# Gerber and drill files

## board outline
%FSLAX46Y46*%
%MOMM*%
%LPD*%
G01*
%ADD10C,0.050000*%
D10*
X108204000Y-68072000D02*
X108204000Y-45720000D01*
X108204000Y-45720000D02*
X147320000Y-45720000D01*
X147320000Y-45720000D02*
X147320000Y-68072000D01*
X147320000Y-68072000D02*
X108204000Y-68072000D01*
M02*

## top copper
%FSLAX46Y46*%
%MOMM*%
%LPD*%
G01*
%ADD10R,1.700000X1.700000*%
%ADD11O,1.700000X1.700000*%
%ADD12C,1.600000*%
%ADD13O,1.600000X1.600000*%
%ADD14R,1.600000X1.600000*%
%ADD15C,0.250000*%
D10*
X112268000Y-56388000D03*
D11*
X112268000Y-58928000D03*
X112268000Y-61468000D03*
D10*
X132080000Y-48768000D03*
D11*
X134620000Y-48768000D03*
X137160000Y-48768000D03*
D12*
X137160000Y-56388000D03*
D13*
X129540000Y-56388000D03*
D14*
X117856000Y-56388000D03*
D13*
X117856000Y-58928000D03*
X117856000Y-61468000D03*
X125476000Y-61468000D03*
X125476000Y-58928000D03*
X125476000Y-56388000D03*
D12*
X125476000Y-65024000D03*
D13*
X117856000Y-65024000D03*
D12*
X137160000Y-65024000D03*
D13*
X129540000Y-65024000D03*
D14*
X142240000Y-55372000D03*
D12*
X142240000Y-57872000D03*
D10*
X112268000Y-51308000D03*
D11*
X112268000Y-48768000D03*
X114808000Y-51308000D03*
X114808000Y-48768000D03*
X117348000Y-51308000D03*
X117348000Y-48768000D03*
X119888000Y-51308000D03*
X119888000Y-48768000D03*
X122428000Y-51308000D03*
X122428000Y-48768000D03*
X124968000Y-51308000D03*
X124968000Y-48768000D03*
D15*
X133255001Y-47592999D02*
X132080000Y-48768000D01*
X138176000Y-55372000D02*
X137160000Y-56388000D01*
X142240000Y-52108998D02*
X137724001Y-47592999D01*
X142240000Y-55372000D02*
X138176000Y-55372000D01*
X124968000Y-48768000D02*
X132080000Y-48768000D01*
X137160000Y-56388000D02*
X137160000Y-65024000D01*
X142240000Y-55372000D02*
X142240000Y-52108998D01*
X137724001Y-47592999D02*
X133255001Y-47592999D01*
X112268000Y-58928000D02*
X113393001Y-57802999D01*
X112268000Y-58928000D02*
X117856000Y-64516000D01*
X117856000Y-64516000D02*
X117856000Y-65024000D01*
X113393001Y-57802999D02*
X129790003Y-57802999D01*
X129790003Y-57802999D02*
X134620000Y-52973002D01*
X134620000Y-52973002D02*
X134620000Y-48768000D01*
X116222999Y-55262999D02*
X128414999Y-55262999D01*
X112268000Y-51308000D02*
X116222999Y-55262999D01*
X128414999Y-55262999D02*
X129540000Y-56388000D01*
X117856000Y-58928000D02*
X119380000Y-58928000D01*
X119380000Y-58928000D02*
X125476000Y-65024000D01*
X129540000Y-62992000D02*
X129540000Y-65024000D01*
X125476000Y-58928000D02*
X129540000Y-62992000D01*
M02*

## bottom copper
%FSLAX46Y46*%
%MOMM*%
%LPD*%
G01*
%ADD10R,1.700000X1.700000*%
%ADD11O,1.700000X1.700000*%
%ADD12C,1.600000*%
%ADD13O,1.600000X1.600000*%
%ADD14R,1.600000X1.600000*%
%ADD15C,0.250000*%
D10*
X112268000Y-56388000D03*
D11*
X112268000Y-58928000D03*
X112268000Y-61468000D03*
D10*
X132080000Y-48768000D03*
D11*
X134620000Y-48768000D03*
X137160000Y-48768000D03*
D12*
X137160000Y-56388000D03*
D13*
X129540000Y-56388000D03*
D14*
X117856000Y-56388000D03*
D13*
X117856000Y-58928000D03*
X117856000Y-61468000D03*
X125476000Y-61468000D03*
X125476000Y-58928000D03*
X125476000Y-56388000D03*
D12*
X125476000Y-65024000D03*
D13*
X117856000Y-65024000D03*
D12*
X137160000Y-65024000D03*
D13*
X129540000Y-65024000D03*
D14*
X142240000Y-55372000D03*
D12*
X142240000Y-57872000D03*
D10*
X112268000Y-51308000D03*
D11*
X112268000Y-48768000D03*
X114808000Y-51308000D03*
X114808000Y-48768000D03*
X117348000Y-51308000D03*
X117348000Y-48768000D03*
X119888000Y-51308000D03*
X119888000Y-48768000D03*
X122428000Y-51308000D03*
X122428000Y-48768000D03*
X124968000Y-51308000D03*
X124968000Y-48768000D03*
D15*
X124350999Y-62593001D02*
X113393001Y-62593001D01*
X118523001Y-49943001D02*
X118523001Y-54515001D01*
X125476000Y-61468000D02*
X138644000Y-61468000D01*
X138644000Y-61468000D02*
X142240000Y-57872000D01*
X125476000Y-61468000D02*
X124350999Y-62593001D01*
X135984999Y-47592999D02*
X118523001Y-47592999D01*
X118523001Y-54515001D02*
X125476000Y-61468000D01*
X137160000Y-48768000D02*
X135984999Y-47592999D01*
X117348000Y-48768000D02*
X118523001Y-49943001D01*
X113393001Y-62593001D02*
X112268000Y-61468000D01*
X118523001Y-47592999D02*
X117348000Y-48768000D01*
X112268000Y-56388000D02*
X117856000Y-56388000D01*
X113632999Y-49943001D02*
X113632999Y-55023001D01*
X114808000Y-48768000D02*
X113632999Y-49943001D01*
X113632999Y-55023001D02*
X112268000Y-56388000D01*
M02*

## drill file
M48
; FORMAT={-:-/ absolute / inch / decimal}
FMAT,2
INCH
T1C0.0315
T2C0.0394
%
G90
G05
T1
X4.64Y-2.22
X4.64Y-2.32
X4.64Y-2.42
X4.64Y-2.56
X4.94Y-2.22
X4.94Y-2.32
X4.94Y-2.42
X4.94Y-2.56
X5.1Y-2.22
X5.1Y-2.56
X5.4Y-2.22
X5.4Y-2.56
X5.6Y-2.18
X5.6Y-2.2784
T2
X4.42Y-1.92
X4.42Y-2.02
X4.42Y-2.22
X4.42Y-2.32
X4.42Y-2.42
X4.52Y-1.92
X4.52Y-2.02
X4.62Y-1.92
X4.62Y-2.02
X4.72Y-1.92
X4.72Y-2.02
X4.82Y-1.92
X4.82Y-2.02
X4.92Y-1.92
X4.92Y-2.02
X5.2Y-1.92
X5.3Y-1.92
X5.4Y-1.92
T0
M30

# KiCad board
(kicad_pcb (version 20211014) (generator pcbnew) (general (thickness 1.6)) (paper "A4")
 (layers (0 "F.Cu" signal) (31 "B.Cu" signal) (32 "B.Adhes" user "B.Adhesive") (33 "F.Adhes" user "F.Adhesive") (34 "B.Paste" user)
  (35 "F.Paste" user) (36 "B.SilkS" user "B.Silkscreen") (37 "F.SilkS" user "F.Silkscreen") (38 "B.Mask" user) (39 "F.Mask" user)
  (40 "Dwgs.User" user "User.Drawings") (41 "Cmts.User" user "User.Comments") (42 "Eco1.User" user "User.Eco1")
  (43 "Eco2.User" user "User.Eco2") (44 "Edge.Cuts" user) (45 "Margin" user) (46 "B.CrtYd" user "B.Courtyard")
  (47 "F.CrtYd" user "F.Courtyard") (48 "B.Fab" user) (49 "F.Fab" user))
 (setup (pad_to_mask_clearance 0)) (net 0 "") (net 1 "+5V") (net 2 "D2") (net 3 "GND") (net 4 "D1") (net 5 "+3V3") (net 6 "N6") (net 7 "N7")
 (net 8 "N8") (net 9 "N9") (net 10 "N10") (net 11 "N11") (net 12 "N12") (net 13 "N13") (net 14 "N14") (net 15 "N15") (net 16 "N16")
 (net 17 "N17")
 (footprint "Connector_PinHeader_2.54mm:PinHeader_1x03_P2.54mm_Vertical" (layer "F.Cu") (at 112.268 56.388)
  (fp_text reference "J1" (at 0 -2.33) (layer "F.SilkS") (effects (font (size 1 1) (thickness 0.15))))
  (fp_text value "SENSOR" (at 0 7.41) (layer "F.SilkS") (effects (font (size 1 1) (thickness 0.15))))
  (pad "1" thru_hole rect locked (at 0 0) (size 1.7 1.7) (drill 1) (layers *.Cu *.Mask) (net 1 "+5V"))
  (pad "2" thru_hole oval locked (at 0 2.54) (size 1.7 1.7) (drill 1) (layers *.Cu *.Mask) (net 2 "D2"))
  (pad "3" thru_hole oval locked (at 0 5.08) (size 1.7 1.7) (drill 1) (layers *.Cu *.Mask) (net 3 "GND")))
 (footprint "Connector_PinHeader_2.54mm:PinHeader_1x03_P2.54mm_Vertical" (layer "F.Cu") (at 132.08 48.768 90)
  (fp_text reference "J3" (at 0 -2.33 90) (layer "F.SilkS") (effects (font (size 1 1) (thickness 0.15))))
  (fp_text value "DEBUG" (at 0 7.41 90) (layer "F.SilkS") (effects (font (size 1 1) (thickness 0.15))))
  (pad "1" thru_hole rect locked (at 0 0 90) (size 1.7 1.7) (drill 1) (layers *.Cu *.Mask) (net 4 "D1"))
  (pad "2" thru_hole oval locked (at 0 2.54 90) (size 1.7 1.7) (drill 1) (layers *.Cu *.Mask) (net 2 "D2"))
  (pad "3" thru_hole oval locked (at 0 5.08 90) (size 1.7 1.7) (drill 1) (layers *.Cu *.Mask) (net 3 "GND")))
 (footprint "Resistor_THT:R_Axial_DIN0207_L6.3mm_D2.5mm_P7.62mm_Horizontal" (layer "F.Cu") (at 137.16 56.388 180)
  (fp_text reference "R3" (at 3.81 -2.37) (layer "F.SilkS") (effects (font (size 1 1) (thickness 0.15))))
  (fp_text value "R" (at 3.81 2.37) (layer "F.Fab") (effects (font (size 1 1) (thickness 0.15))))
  (pad "1" thru_hole circle locked (at 0 0 180) (size 1.6 1.6) (drill 0.8) (layers *.Cu *.Mask) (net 4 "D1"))
  (pad "2" thru_hole oval locked (at 7.62 0 180) (size 1.6 1.6) (drill 0.8) (layers *.Cu *.Mask) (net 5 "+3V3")))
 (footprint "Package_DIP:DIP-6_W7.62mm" (layer "F.Cu") (at 117.856 56.388)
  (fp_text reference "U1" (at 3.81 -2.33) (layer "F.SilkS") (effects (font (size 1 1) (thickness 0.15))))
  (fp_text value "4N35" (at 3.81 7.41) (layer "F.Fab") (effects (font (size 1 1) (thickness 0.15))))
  (pad "1" thru_hole rect locked (at 0 0) (size 1.6 1.6) (drill 0.8) (layers *.Cu *.Mask) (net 1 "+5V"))
  (pad "2" thru_hole oval locked (at 0 2.54) (size 1.6 1.6) (drill 0.8) (layers *.Cu *.Mask) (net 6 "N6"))
  (pad "3" thru_hole oval locked (at 0 5.08) (size 1.6 1.6) (drill 0.8) (layers *.Cu *.Mask) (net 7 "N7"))
  (pad "4" thru_hole oval locked (at 7.62 5.08) (size 1.6 1.6) (drill 0.8) (layers *.Cu *.Mask) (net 3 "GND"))
  (pad "5" thru_hole oval locked (at 7.62 2.54) (size 1.6 1.6) (drill 0.8) (layers *.Cu *.Mask) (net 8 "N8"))
  (pad "6" thru_hole oval locked (at 7.62 0) (size 1.6 1.6) (drill 0.8) (layers *.Cu *.Mask) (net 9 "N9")))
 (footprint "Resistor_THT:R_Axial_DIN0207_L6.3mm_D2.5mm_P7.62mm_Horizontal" (layer "F.Cu") (at 125.476 65.024 180)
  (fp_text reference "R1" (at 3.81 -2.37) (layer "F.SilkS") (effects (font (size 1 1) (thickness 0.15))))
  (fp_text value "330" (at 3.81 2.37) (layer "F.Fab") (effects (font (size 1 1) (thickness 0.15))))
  (pad "1" thru_hole circle locked (at 0 0 180) (size 1.6 1.6) (drill 0.8) (layers *.Cu *.Mask) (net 6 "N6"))
  (pad "2" thru_hole oval locked (at 7.62 0 180) (size 1.6 1.6) (drill 0.8) (layers *.Cu *.Mask) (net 2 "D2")))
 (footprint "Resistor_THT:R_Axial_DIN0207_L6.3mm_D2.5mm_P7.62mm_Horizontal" (layer "F.Cu") (at 137.16 65.024 180)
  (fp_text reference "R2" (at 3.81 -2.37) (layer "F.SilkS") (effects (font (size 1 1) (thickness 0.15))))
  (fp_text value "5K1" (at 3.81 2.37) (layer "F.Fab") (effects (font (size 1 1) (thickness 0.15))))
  (pad "1" thru_hole circle locked (at 0 0 180) (size 1.6 1.6) (drill 0.8) (layers *.Cu *.Mask) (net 4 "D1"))
  (pad "2" thru_hole oval locked (at 7.62 0 180) (size 1.6 1.6) (drill 0.8) (layers *.Cu *.Mask) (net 8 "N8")))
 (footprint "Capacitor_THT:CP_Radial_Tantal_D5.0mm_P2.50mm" (layer "F.Cu") (at 142.24 55.372 -90)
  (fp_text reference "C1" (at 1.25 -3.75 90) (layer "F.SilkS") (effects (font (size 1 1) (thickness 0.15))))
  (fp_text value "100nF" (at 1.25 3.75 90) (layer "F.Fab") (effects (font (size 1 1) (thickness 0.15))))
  (pad "1" thru_hole rect locked (at 0 0 270) (size 1.6 1.6) (drill 0.8) (layers *.Cu *.Mask) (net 4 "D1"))
  (pad "2" thru_hole circle locked (at 2.5 0 270) (size 1.6 1.6) (drill 0.8) (layers *.Cu *.Mask) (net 3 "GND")))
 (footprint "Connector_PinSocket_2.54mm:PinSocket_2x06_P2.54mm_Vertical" (layer "B.Cu") (at 112.268 51.308 -90)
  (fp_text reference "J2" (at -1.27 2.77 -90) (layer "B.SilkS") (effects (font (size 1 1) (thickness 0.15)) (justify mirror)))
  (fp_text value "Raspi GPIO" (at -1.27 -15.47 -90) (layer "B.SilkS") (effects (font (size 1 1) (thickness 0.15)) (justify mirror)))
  (pad "1" thru_hole rect locked (at 0 0 270) (size 1.7 1.7) (drill 1) (layers *.Cu *.Mask) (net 5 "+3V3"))
  (pad "2" thru_hole oval locked (at -2.54 0 270) (size 1.7 1.7) (drill 1) (layers *.Cu *.Mask) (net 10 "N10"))
  (pad "3" thru_hole oval locked (at 0 -2.54 270) (size 1.7 1.7) (drill 1) (layers *.Cu *.Mask) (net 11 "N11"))
  (pad "4" thru_hole oval locked (at -2.54 -2.54 270) (size 1.7 1.7) (drill 1) (layers *.Cu *.Mask) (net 1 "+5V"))
  (pad "5" thru_hole oval locked (at 0 -5.08 270) (size 1.7 1.7) (drill 1) (layers *.Cu *.Mask) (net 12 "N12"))
  (pad "6" thru_hole oval locked (at -2.54 -5.08 270) (size 1.7 1.7) (drill 1) (layers *.Cu *.Mask) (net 3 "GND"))
  (pad "7" thru_hole oval locked (at 0 -7.62 270) (size 1.7 1.7) (drill 1) (layers *.Cu *.Mask) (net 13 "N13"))
  (pad "8" thru_hole oval locked (at -2.54 -7.62 270) (size 1.7 1.7) (drill 1) (layers *.Cu *.Mask) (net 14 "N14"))
  (pad "9" thru_hole oval locked (at 0 -10.16 270) (size 1.7 1.7) (drill 1) (layers *.Cu *.Mask) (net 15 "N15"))
  (pad "10" thru_hole oval locked (at -2.54 -10.16 270) (size 1.7 1.7) (drill 1) (layers *.Cu *.Mask) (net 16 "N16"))
  (pad "11" thru_hole oval locked (at 0 -12.7 270) (size 1.7 1.7) (drill 1) (layers *.Cu *.Mask) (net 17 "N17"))
  (pad "12" thru_hole oval locked (at -2.54 -12.7 270) (size 1.7 1.7) (drill 1) (layers *.Cu *.Mask) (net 4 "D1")))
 (gr_line (start 108.204 68.072) (end 108.204 45.72) (layer "Edge.Cuts") (width 0.05))
 (gr_line (start 108.204 45.72) (end 147.32 45.72) (layer "Edge.Cuts") (width 0.05))
 (gr_line (start 147.32 45.72) (end 147.32 68.072) (layer "Edge.Cuts") (width 0.05))
 (gr_line (start 147.32 68.072) (end 108.204 68.072) (layer "Edge.Cuts") (width 0.05))
 (segment (start 124.350999 62.593001) (end 113.393001 62.593001) (width 0.25) (layer "B.Cu") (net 3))
 (segment (start 118.523001 49.943001) (end 118.523001 54.515001) (width 0.25) (layer "B.Cu") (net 3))
 (segment (start 125.476 61.468) (end 138.644 61.468) (width 0.25) (layer "B.Cu") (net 3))
 (segment (start 138.644 61.468) (end 142.24 57.872) (width 0.25) (layer "B.Cu") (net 3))
 (segment (start 125.476 61.468) (end 124.350999 62.593001) (width 0.25) (layer "B.Cu") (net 3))
 (segment (start 135.984999 47.592999) (end 118.523001 47.592999) (width 0.25) (layer "B.Cu") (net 3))
 (segment (start 118.523001 54.515001) (end 125.476 61.468) (width 0.25) (layer "B.Cu") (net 3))
 (segment (start 137.16 48.768) (end 135.984999 47.592999) (width 0.25) (layer "B.Cu") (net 3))
 (segment (start 117.348 48.768) (end 118.523001 49.943001) (width 0.25) (layer "B.Cu") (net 3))
 (segment (start 113.393001 62.593001) (end 112.268 61.468) (width 0.25) (layer "B.Cu") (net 3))
 (segment (start 118.523001 47.592999) (end 117.348 48.768) (width 0.25) (layer "B.Cu") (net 3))
 (segment (start 133.255001 47.592999) (end 132.08 48.768) (width 0.25) (layer "F.Cu") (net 4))
 (segment (start 138.176 55.372) (end 137.16 56.388) (width 0.25) (layer "F.Cu") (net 4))
 (segment (start 142.24 52.108998) (end 137.724001 47.592999) (width 0.25) (layer "F.Cu") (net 4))
 (segment (start 142.24 55.372) (end 138.176 55.372) (width 0.25) (layer "F.Cu") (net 4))
 (segment (start 124.968 48.768) (end 132.08 48.768) (width 0.25) (layer "F.Cu") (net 4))
 (segment (start 137.16 56.388) (end 137.16 65.024) (width 0.25) (layer "F.Cu") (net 4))
 (segment (start 142.24 55.372) (end 142.24 52.108998) (width 0.25) (layer "F.Cu") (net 4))
 (segment (start 137.724001 47.592999) (end 133.255001 47.592999) (width 0.25) (layer "F.Cu") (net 4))
 (segment (start 112.268 58.928) (end 113.393001 57.802999) (width 0.25) (layer "F.Cu") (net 2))
 (segment (start 112.268 58.928) (end 117.856 64.516) (width 0.25) (layer "F.Cu") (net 2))
 (segment (start 117.856 64.516) (end 117.856 65.024) (width 0.25) (layer "F.Cu") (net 2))
 (segment (start 113.393001 57.802999) (end 129.790003 57.802999) (width 0.25) (layer "F.Cu") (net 2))
 (segment (start 129.790003 57.802999) (end 134.62 52.973002) (width 0.25) (layer "F.Cu") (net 2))
 (segment (start 134.62 52.973002) (end 134.62 48.768) (width 0.25) (layer "F.Cu") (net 2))
 (segment (start 112.268 56.388) (end 117.856 56.388) (width 0.25) (layer "B.Cu") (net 1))
 (segment (start 113.632999 49.943001) (end 113.632999 55.023001) (width 0.25) (layer "B.Cu") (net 1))
 (segment (start 114.808 48.768) (end 113.632999 49.943001) (width 0.25) (layer "B.Cu") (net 1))
 (segment (start 113.632999 55.023001) (end 112.268 56.388) (width 0.25) (layer "B.Cu") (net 1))
 (segment (start 116.222999 55.262999) (end 128.414999 55.262999) (width 0.25) (layer "F.Cu") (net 5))
 (segment (start 112.268 51.308) (end 116.222999 55.262999) (width 0.25) (layer "F.Cu") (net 5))
 (segment (start 128.414999 55.262999) (end 129.54 56.388) (width 0.25) (layer "F.Cu") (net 5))
 (segment (start 117.856 58.928) (end 119.38 58.928) (width 0.25) (layer "F.Cu") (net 6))
 (segment (start 119.38 58.928) (end 125.476 65.024) (width 0.25) (layer "F.Cu") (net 6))
 (segment (start 129.54 62.992) (end 129.54 65.024) (width 0.25) (layer "F.Cu") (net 8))
 (segment (start 125.476 58.928) (end 129.54 62.992) (width 0.25) (layer "F.Cu") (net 8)))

